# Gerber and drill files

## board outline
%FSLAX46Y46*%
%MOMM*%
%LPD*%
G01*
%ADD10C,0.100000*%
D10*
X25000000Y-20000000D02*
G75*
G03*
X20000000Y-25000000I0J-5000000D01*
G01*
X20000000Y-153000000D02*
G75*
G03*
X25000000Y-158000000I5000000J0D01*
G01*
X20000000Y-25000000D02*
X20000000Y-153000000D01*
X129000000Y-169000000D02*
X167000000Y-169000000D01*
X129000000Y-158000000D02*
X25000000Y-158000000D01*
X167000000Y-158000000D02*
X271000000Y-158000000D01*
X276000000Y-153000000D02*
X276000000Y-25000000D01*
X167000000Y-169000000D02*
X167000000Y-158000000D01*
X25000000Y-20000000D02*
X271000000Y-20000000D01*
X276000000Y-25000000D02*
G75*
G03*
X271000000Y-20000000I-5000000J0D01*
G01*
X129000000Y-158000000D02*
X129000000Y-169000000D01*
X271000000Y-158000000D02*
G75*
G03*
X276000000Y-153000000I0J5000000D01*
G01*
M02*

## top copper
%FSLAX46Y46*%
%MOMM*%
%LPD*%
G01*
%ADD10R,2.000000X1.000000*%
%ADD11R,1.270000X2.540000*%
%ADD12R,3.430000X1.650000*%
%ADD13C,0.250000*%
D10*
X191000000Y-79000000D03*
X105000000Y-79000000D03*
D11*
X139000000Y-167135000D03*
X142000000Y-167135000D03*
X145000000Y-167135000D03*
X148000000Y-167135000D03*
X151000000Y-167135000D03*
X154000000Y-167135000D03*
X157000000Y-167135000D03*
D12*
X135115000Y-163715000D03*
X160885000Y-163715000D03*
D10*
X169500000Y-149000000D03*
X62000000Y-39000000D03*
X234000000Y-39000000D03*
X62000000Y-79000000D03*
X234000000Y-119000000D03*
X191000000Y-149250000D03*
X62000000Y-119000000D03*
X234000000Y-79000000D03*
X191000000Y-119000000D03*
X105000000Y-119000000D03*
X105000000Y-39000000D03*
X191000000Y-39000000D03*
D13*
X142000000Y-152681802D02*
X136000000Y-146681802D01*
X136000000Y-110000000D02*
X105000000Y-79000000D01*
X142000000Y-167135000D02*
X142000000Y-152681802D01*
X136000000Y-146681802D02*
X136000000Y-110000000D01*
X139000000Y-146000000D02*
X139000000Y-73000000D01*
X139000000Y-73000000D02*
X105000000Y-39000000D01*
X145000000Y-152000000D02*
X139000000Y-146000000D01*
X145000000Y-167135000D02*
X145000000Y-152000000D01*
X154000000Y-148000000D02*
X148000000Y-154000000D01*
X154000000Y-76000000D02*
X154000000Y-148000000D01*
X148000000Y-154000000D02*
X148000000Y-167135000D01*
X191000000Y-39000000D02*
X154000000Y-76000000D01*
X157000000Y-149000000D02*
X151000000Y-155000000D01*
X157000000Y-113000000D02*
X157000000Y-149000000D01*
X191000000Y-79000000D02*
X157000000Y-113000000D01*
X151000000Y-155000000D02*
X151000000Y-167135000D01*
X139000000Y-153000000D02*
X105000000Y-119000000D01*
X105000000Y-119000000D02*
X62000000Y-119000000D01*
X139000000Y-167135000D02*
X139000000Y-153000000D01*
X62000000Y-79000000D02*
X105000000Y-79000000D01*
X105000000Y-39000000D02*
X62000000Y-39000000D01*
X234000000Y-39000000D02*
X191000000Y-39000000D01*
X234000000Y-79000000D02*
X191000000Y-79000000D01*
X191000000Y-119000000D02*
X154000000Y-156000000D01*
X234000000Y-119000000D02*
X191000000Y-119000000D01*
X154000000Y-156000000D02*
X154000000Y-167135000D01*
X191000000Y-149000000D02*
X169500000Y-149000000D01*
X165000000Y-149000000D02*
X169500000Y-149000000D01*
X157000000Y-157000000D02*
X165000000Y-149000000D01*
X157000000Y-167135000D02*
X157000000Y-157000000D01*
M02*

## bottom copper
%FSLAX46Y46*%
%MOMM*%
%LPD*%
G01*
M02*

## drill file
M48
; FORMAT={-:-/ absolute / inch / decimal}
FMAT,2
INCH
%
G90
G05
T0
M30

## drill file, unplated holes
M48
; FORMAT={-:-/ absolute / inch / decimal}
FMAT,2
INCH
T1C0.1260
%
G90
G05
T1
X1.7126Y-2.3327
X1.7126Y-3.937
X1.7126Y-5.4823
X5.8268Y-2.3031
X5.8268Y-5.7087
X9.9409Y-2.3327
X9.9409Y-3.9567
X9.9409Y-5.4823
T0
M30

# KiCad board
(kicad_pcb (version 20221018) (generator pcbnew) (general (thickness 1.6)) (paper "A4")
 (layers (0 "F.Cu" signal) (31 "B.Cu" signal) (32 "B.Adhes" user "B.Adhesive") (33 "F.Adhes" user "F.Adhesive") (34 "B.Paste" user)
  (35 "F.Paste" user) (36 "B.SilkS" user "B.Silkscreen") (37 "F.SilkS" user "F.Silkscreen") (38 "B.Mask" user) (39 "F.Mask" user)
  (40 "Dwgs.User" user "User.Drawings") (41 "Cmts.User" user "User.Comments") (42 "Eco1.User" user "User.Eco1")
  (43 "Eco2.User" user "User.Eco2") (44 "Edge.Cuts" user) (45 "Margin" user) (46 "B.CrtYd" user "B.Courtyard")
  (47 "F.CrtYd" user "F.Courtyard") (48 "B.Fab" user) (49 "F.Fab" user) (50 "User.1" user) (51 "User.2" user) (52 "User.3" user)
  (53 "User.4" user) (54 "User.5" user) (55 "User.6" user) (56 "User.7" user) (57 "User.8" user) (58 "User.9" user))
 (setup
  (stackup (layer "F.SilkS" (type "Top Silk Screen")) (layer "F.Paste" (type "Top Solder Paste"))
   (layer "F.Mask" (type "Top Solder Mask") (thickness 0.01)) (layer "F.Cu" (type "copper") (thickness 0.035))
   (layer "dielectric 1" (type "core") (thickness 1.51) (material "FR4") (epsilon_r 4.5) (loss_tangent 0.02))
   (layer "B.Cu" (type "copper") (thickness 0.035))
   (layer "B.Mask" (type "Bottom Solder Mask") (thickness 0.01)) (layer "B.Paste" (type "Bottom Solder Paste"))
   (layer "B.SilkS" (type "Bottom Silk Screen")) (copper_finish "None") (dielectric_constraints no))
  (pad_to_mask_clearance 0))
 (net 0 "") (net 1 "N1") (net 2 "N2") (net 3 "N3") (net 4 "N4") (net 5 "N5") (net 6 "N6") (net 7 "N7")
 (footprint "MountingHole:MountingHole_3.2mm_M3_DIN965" (layer "F.Cu") (at 43.5 100)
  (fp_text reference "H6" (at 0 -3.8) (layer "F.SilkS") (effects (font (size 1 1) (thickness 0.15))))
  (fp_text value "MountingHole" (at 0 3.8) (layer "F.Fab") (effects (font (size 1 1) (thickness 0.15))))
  (pad "" np_thru_hole circle (at 0 0) (size 3.2 3.2) (drill 3.2) (layers "*.Cu" "*.Mask")))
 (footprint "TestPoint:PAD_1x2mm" (layer "F.Cu") (at 191 79)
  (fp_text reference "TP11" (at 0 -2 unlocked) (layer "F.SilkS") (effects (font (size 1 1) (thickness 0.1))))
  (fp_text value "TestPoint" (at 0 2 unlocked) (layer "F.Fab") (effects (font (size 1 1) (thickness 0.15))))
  (pad "1" smd rect (at 0 0 90) (size 1 2) (layers "F.Cu" "F.Paste" "F.Mask") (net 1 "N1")))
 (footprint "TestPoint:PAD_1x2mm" (layer "F.Cu") (at 105 79)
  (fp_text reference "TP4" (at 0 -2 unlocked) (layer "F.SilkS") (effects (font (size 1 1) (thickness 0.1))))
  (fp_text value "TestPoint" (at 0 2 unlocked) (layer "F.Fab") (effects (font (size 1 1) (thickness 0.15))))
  (pad "1" smd rect (at 0 0 90) (size 1 2) (layers "F.Cu" "F.Paste" "F.Mask") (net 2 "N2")))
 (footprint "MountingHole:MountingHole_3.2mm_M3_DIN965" (layer "F.Cu") (at 252.5 139.25)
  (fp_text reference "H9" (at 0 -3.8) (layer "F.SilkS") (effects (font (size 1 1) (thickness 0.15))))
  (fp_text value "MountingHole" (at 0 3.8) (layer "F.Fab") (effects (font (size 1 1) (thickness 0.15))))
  (pad "" np_thru_hole circle (at 0 0) (size 3.2 3.2) (drill 3.2) (layers "*.Cu" "*.Mask")))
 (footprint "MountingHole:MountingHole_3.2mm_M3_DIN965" (layer "F.Cu") (at 148 58.5)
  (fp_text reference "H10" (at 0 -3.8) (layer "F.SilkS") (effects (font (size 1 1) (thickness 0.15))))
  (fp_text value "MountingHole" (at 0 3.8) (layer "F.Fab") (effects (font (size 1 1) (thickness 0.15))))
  (pad "" np_thru_hole circle (at 0 0) (size 3.2 3.2) (drill 3.2) (layers "*.Cu" "*.Mask")))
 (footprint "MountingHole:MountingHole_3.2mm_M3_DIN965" (layer "F.Cu") (at 43.5 139.25)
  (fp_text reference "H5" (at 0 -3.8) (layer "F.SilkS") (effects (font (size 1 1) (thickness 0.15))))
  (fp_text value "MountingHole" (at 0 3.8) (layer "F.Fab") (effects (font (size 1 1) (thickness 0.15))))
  (pad "" np_thru_hole circle (at 0 0) (size 3.2 3.2) (drill 3.2) (layers "*.Cu" "*.Mask")))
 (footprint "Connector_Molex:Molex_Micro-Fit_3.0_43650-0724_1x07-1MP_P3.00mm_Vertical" (layer "F.Cu") (at 148 164)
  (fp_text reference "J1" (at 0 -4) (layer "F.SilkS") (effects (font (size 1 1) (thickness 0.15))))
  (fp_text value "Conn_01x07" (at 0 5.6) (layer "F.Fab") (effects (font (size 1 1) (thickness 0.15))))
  (pad "1" smd rect (at -9 3.135) (size 1.27 2.54) (layers "F.Cu" "F.Paste" "F.Mask") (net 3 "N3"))
  (pad "2" smd rect (at -6 3.135) (size 1.27 2.54) (layers "F.Cu" "F.Paste" "F.Mask") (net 2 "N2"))
  (pad "3" smd rect (at -3 3.135) (size 1.27 2.54) (layers "F.Cu" "F.Paste" "F.Mask") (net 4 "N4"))
  (pad "4" smd rect (at 0 3.135) (size 1.27 2.54) (layers "F.Cu" "F.Paste" "F.Mask") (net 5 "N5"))
  (pad "5" smd rect (at 3 3.135) (size 1.27 2.54) (layers "F.Cu" "F.Paste" "F.Mask") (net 1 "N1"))
  (pad "6" smd rect (at 6 3.135) (size 1.27 2.54) (layers "F.Cu" "F.Paste" "F.Mask") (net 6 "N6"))
  (pad "7" smd rect (at 9 3.135) (size 1.27 2.54) (layers "F.Cu" "F.Paste" "F.Mask") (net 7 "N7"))
  (pad "MP" smd rect (at -12.885 -0.285) (size 3.43 1.65) (layers "F.Cu" "F.Paste" "F.Mask"))
  (pad "MP" smd rect (at 12.885 -0.285) (size 3.43 1.65) (layers "F.Cu" "F.Paste" "F.Mask")))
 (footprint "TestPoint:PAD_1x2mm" (layer "F.Cu") (at 169.5 149)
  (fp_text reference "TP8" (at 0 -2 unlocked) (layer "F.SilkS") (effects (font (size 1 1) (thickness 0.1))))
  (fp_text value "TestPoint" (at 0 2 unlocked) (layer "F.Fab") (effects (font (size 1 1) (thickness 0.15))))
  (pad "1" smd rect (at 0 0 90) (size 1 2) (layers "F.Cu" "F.Paste" "F.Mask") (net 7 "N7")))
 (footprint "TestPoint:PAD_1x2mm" (layer "F.Cu") (at 62 39)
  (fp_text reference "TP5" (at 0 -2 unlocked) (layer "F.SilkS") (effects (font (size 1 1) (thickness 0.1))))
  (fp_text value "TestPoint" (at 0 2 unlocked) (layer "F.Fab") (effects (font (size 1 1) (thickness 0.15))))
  (pad "1" smd rect (at 0 0 90) (size 1 2) (layers "F.Cu" "F.Paste" "F.Mask") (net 4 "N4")))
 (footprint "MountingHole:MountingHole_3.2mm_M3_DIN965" (layer "F.Cu") (at 252.5 59.25)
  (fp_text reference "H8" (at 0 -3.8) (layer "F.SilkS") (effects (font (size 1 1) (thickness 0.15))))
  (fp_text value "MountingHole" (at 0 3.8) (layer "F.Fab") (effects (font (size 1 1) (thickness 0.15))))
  (pad "" np_thru_hole circle (at 0 0) (size 3.2 3.2) (drill 3.2) (layers "*.Cu" "*.Mask")))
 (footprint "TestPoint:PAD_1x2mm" (layer "F.Cu") (at 234 39)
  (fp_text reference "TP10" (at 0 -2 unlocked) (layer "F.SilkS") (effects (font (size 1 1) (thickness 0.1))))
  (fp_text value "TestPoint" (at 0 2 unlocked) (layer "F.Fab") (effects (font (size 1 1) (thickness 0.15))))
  (pad "1" smd rect (at 0 0 90) (size 1 2) (layers "F.Cu" "F.Paste" "F.Mask") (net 5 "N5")))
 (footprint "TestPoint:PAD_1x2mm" (layer "F.Cu") (at 62 79)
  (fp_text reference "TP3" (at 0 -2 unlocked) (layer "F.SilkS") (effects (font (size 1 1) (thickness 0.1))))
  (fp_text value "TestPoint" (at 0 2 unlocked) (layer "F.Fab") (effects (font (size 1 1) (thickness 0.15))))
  (pad "1" smd rect (at 0 0 90) (size 1 2) (layers "F.Cu" "F.Paste" "F.Mask") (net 2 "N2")))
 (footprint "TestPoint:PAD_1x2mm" (layer "F.Cu") (at 234 119)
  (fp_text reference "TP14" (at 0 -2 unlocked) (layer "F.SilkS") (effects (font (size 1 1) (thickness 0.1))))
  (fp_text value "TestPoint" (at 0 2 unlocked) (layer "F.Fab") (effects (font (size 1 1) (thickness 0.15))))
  (pad "1" smd rect (at 0 0 90) (size 1 2) (layers "F.Cu" "F.Paste" "F.Mask") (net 6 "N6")))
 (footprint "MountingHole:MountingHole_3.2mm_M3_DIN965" (layer "F.Cu") (at 148 145)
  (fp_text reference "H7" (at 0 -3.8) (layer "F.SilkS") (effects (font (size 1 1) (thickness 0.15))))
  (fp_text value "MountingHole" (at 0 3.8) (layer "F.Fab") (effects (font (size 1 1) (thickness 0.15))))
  (pad "" np_thru_hole circle (at 0 0) (size 3.2 3.2) (drill 3.2) (layers "*.Cu" "*.Mask")))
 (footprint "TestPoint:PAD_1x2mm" (layer "F.Cu") (at 191 149.25)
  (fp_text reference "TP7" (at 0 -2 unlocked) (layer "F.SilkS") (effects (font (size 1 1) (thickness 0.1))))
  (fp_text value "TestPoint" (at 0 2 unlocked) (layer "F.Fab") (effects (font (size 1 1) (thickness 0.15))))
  (pad "1" smd rect (at 0 0 90) (size 1 2) (layers "F.Cu" "F.Paste" "F.Mask") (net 7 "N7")))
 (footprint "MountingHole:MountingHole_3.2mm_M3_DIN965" (layer "F.Cu") (at 252.5 100.5)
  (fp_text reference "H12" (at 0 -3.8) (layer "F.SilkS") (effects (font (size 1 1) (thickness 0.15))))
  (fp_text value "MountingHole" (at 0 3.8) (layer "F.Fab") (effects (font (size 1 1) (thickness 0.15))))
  (pad "" np_thru_hole circle (at 0 0) (size 3.2 3.2) (drill 3.2) (layers "*.Cu" "*.Mask")))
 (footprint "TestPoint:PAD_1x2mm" (layer "F.Cu") (at 62 119)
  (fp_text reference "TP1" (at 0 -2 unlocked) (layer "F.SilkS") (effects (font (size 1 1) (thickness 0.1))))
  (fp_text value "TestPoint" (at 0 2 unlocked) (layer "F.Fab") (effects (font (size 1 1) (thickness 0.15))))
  (pad "1" smd rect (at 0 0 90) (size 1 2) (layers "F.Cu" "F.Paste" "F.Mask") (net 3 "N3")))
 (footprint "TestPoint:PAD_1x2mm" (layer "F.Cu") (at 234 79)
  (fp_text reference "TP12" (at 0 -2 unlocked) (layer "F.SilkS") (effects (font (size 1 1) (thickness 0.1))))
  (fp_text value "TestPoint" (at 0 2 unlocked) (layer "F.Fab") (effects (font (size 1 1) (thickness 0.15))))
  (pad "1" smd rect (at 0 0 90) (size 1 2) (layers "F.Cu" "F.Paste" "F.Mask") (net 1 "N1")))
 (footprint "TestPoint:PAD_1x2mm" (layer "F.Cu") (at 191 119)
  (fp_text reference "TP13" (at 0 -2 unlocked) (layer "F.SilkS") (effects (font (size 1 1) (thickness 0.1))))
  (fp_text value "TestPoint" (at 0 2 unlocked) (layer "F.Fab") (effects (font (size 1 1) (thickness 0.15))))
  (pad "1" smd rect (at 0 0 90) (size 1 2) (layers "F.Cu" "F.Paste" "F.Mask") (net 6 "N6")))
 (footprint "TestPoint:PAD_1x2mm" (layer "F.Cu") (at 105 119)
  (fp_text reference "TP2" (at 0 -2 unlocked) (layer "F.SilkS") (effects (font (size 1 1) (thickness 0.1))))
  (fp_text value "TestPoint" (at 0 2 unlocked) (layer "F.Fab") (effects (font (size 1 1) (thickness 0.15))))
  (pad "1" smd rect (at 0 0 90) (size 1 2) (layers "F.Cu" "F.Paste" "F.Mask") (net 3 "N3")))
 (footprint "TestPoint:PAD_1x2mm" (layer "F.Cu") (at 105 39)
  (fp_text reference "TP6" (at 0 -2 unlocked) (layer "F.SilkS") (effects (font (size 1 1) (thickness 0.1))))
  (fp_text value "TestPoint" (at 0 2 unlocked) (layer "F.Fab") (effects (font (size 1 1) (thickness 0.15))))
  (pad "1" smd rect (at 0 0 90) (size 1 2) (layers "F.Cu" "F.Paste" "F.Mask") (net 4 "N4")))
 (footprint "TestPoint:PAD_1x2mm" (layer "F.Cu") (at 191 39)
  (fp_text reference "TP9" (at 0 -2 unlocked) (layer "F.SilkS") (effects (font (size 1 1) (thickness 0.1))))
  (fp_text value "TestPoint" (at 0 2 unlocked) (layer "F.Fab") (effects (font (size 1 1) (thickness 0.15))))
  (pad "1" smd rect (at 0 0 90) (size 1 2) (layers "F.Cu" "F.Paste" "F.Mask") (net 5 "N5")))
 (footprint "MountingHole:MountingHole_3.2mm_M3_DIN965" (layer "F.Cu") (at 43.5 59.25)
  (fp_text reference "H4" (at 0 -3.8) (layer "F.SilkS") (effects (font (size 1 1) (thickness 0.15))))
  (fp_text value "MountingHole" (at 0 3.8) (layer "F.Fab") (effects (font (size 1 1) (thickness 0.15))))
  (pad "" np_thru_hole circle (at 0 0) (size 3.2 3.2) (drill 3.2) (layers "*.Cu" "*.Mask")))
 (gr_arc (start 20 25) (mid 21.464466 21.464466) (end 25 20) (stroke (width 0.1) (type default)) (layer "Edge.Cuts"))
 (gr_arc (start 25 158) (mid 21.464466 156.535534) (end 20 153) (stroke (width 0.1) (type default)) (layer "Edge.Cuts"))
 (gr_line (start 20 25) (end 20 153) (stroke (width 0.1) (type default)) (layer "Edge.Cuts"))
 (gr_line (start 129 169) (end 167 169) (stroke (width 0.1) (type default)) (layer "Edge.Cuts"))
 (gr_line (start 129 158) (end 25 158) (stroke (width 0.1) (type default)) (layer "Edge.Cuts"))
 (gr_line (start 167 158) (end 271 158) (stroke (width 0.1) (type default)) (layer "Edge.Cuts"))
 (gr_line (start 276 153) (end 276 25) (stroke (width 0.1) (type default)) (layer "Edge.Cuts"))
 (gr_line (start 167 169) (end 167 158) (stroke (width 0.1) (type default)) (layer "Edge.Cuts"))
 (gr_line (start 25 20) (end 271 20) (stroke (width 0.1) (type default)) (layer "Edge.Cuts"))
 (gr_arc (start 271 20) (mid 274.535534 21.464466) (end 276 25) (stroke (width 0.1) (type default)) (layer "Edge.Cuts"))
 (gr_line (start 129 158) (end 129 169) (stroke (width 0.1) (type default)) (layer "Edge.Cuts"))
 (gr_arc (start 276 153) (mid 274.535534 156.535534) (end 271 158) (stroke (width 0.1) (type default)) (layer "Edge.Cuts"))
 (segment (start 139 153) (end 105 119) (width 0.25) (layer "F.Cu") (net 3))
 (segment (start 105 119) (end 62 119) (width 0.25) (layer "F.Cu") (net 3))
 (segment (start 139 167.135) (end 139 153) (width 0.25) (layer "F.Cu") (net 3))
 (segment (start 136 110) (end 105 79) (width 0.25) (layer "F.Cu") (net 2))
 (segment (start 142 152.681802) (end 136 146.681802) (width 0.25) (layer "F.Cu") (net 2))
 (segment (start 62 79) (end 105 79) (width 0.25) (layer "F.Cu") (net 2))
 (segment (start 136 146.681802) (end 136 110) (width 0.25) (layer "F.Cu") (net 2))
 (segment (start 142 167.135) (end 142 152.681802) (width 0.25) (layer "F.Cu") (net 2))
 (segment (start 145 167.135) (end 145 152) (width 0.25) (layer "F.Cu") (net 4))
 (segment (start 139 73) (end 105 39) (width 0.25) (layer "F.Cu") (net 4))
 (segment (start 145 152) (end 139 146) (width 0.25) (layer "F.Cu") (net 4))
 (segment (start 139 146) (end 139 73) (width 0.25) (layer "F.Cu") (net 4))
 (segment (start 105 39) (end 62 39) (width 0.25) (layer "F.Cu") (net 4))
 (segment (start 191 39) (end 154 76) (width 0.25) (layer "F.Cu") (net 5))
 (segment (start 154 76) (end 154 148) (width 0.25) (layer "F.Cu") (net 5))
 (segment (start 234 39) (end 191 39) (width 0.25) (layer "F.Cu") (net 5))
 (segment (start 154 148) (end 148 154) (width 0.25) (layer "F.Cu") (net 5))
 (segment (start 148 154) (end 148 167.135) (width 0.25) (layer "F.Cu") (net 5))
 (segment (start 157 113) (end 157 149) (width 0.25) (layer "F.Cu") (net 1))
 (segment (start 234 79) (end 191 79) (width 0.25) (layer "F.Cu") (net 1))
 (segment (start 191 79) (end 157 113) (width 0.25) (layer "F.Cu") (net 1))
 (segment (start 157 149) (end 151 155) (width 0.25) (layer "F.Cu") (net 1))
 (segment (start 151 155) (end 151 167.135) (width 0.25) (layer "F.Cu") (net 1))
 (segment (start 191 119) (end 154 156) (width 0.25) (layer "F.Cu") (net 6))
 (segment (start 234 119) (end 191 119) (width 0.25) (layer "F.Cu") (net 6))
 (segment (start 154 156) (end 154 167.135) (width 0.25) (layer "F.Cu") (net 6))
 (segment (start 191 149) (end 169.5 149) (width 0.25) (layer "F.Cu") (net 7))
 (segment (start 165 149) (end 169.5 149) (width 0.25) (layer "F.Cu") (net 7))
 (segment (start 157 157) (end 165 149) (width 0.25) (layer "F.Cu") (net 7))
 (segment (start 157 167.135) (end 157 157) (width 0.25) (layer "F.Cu") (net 7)))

